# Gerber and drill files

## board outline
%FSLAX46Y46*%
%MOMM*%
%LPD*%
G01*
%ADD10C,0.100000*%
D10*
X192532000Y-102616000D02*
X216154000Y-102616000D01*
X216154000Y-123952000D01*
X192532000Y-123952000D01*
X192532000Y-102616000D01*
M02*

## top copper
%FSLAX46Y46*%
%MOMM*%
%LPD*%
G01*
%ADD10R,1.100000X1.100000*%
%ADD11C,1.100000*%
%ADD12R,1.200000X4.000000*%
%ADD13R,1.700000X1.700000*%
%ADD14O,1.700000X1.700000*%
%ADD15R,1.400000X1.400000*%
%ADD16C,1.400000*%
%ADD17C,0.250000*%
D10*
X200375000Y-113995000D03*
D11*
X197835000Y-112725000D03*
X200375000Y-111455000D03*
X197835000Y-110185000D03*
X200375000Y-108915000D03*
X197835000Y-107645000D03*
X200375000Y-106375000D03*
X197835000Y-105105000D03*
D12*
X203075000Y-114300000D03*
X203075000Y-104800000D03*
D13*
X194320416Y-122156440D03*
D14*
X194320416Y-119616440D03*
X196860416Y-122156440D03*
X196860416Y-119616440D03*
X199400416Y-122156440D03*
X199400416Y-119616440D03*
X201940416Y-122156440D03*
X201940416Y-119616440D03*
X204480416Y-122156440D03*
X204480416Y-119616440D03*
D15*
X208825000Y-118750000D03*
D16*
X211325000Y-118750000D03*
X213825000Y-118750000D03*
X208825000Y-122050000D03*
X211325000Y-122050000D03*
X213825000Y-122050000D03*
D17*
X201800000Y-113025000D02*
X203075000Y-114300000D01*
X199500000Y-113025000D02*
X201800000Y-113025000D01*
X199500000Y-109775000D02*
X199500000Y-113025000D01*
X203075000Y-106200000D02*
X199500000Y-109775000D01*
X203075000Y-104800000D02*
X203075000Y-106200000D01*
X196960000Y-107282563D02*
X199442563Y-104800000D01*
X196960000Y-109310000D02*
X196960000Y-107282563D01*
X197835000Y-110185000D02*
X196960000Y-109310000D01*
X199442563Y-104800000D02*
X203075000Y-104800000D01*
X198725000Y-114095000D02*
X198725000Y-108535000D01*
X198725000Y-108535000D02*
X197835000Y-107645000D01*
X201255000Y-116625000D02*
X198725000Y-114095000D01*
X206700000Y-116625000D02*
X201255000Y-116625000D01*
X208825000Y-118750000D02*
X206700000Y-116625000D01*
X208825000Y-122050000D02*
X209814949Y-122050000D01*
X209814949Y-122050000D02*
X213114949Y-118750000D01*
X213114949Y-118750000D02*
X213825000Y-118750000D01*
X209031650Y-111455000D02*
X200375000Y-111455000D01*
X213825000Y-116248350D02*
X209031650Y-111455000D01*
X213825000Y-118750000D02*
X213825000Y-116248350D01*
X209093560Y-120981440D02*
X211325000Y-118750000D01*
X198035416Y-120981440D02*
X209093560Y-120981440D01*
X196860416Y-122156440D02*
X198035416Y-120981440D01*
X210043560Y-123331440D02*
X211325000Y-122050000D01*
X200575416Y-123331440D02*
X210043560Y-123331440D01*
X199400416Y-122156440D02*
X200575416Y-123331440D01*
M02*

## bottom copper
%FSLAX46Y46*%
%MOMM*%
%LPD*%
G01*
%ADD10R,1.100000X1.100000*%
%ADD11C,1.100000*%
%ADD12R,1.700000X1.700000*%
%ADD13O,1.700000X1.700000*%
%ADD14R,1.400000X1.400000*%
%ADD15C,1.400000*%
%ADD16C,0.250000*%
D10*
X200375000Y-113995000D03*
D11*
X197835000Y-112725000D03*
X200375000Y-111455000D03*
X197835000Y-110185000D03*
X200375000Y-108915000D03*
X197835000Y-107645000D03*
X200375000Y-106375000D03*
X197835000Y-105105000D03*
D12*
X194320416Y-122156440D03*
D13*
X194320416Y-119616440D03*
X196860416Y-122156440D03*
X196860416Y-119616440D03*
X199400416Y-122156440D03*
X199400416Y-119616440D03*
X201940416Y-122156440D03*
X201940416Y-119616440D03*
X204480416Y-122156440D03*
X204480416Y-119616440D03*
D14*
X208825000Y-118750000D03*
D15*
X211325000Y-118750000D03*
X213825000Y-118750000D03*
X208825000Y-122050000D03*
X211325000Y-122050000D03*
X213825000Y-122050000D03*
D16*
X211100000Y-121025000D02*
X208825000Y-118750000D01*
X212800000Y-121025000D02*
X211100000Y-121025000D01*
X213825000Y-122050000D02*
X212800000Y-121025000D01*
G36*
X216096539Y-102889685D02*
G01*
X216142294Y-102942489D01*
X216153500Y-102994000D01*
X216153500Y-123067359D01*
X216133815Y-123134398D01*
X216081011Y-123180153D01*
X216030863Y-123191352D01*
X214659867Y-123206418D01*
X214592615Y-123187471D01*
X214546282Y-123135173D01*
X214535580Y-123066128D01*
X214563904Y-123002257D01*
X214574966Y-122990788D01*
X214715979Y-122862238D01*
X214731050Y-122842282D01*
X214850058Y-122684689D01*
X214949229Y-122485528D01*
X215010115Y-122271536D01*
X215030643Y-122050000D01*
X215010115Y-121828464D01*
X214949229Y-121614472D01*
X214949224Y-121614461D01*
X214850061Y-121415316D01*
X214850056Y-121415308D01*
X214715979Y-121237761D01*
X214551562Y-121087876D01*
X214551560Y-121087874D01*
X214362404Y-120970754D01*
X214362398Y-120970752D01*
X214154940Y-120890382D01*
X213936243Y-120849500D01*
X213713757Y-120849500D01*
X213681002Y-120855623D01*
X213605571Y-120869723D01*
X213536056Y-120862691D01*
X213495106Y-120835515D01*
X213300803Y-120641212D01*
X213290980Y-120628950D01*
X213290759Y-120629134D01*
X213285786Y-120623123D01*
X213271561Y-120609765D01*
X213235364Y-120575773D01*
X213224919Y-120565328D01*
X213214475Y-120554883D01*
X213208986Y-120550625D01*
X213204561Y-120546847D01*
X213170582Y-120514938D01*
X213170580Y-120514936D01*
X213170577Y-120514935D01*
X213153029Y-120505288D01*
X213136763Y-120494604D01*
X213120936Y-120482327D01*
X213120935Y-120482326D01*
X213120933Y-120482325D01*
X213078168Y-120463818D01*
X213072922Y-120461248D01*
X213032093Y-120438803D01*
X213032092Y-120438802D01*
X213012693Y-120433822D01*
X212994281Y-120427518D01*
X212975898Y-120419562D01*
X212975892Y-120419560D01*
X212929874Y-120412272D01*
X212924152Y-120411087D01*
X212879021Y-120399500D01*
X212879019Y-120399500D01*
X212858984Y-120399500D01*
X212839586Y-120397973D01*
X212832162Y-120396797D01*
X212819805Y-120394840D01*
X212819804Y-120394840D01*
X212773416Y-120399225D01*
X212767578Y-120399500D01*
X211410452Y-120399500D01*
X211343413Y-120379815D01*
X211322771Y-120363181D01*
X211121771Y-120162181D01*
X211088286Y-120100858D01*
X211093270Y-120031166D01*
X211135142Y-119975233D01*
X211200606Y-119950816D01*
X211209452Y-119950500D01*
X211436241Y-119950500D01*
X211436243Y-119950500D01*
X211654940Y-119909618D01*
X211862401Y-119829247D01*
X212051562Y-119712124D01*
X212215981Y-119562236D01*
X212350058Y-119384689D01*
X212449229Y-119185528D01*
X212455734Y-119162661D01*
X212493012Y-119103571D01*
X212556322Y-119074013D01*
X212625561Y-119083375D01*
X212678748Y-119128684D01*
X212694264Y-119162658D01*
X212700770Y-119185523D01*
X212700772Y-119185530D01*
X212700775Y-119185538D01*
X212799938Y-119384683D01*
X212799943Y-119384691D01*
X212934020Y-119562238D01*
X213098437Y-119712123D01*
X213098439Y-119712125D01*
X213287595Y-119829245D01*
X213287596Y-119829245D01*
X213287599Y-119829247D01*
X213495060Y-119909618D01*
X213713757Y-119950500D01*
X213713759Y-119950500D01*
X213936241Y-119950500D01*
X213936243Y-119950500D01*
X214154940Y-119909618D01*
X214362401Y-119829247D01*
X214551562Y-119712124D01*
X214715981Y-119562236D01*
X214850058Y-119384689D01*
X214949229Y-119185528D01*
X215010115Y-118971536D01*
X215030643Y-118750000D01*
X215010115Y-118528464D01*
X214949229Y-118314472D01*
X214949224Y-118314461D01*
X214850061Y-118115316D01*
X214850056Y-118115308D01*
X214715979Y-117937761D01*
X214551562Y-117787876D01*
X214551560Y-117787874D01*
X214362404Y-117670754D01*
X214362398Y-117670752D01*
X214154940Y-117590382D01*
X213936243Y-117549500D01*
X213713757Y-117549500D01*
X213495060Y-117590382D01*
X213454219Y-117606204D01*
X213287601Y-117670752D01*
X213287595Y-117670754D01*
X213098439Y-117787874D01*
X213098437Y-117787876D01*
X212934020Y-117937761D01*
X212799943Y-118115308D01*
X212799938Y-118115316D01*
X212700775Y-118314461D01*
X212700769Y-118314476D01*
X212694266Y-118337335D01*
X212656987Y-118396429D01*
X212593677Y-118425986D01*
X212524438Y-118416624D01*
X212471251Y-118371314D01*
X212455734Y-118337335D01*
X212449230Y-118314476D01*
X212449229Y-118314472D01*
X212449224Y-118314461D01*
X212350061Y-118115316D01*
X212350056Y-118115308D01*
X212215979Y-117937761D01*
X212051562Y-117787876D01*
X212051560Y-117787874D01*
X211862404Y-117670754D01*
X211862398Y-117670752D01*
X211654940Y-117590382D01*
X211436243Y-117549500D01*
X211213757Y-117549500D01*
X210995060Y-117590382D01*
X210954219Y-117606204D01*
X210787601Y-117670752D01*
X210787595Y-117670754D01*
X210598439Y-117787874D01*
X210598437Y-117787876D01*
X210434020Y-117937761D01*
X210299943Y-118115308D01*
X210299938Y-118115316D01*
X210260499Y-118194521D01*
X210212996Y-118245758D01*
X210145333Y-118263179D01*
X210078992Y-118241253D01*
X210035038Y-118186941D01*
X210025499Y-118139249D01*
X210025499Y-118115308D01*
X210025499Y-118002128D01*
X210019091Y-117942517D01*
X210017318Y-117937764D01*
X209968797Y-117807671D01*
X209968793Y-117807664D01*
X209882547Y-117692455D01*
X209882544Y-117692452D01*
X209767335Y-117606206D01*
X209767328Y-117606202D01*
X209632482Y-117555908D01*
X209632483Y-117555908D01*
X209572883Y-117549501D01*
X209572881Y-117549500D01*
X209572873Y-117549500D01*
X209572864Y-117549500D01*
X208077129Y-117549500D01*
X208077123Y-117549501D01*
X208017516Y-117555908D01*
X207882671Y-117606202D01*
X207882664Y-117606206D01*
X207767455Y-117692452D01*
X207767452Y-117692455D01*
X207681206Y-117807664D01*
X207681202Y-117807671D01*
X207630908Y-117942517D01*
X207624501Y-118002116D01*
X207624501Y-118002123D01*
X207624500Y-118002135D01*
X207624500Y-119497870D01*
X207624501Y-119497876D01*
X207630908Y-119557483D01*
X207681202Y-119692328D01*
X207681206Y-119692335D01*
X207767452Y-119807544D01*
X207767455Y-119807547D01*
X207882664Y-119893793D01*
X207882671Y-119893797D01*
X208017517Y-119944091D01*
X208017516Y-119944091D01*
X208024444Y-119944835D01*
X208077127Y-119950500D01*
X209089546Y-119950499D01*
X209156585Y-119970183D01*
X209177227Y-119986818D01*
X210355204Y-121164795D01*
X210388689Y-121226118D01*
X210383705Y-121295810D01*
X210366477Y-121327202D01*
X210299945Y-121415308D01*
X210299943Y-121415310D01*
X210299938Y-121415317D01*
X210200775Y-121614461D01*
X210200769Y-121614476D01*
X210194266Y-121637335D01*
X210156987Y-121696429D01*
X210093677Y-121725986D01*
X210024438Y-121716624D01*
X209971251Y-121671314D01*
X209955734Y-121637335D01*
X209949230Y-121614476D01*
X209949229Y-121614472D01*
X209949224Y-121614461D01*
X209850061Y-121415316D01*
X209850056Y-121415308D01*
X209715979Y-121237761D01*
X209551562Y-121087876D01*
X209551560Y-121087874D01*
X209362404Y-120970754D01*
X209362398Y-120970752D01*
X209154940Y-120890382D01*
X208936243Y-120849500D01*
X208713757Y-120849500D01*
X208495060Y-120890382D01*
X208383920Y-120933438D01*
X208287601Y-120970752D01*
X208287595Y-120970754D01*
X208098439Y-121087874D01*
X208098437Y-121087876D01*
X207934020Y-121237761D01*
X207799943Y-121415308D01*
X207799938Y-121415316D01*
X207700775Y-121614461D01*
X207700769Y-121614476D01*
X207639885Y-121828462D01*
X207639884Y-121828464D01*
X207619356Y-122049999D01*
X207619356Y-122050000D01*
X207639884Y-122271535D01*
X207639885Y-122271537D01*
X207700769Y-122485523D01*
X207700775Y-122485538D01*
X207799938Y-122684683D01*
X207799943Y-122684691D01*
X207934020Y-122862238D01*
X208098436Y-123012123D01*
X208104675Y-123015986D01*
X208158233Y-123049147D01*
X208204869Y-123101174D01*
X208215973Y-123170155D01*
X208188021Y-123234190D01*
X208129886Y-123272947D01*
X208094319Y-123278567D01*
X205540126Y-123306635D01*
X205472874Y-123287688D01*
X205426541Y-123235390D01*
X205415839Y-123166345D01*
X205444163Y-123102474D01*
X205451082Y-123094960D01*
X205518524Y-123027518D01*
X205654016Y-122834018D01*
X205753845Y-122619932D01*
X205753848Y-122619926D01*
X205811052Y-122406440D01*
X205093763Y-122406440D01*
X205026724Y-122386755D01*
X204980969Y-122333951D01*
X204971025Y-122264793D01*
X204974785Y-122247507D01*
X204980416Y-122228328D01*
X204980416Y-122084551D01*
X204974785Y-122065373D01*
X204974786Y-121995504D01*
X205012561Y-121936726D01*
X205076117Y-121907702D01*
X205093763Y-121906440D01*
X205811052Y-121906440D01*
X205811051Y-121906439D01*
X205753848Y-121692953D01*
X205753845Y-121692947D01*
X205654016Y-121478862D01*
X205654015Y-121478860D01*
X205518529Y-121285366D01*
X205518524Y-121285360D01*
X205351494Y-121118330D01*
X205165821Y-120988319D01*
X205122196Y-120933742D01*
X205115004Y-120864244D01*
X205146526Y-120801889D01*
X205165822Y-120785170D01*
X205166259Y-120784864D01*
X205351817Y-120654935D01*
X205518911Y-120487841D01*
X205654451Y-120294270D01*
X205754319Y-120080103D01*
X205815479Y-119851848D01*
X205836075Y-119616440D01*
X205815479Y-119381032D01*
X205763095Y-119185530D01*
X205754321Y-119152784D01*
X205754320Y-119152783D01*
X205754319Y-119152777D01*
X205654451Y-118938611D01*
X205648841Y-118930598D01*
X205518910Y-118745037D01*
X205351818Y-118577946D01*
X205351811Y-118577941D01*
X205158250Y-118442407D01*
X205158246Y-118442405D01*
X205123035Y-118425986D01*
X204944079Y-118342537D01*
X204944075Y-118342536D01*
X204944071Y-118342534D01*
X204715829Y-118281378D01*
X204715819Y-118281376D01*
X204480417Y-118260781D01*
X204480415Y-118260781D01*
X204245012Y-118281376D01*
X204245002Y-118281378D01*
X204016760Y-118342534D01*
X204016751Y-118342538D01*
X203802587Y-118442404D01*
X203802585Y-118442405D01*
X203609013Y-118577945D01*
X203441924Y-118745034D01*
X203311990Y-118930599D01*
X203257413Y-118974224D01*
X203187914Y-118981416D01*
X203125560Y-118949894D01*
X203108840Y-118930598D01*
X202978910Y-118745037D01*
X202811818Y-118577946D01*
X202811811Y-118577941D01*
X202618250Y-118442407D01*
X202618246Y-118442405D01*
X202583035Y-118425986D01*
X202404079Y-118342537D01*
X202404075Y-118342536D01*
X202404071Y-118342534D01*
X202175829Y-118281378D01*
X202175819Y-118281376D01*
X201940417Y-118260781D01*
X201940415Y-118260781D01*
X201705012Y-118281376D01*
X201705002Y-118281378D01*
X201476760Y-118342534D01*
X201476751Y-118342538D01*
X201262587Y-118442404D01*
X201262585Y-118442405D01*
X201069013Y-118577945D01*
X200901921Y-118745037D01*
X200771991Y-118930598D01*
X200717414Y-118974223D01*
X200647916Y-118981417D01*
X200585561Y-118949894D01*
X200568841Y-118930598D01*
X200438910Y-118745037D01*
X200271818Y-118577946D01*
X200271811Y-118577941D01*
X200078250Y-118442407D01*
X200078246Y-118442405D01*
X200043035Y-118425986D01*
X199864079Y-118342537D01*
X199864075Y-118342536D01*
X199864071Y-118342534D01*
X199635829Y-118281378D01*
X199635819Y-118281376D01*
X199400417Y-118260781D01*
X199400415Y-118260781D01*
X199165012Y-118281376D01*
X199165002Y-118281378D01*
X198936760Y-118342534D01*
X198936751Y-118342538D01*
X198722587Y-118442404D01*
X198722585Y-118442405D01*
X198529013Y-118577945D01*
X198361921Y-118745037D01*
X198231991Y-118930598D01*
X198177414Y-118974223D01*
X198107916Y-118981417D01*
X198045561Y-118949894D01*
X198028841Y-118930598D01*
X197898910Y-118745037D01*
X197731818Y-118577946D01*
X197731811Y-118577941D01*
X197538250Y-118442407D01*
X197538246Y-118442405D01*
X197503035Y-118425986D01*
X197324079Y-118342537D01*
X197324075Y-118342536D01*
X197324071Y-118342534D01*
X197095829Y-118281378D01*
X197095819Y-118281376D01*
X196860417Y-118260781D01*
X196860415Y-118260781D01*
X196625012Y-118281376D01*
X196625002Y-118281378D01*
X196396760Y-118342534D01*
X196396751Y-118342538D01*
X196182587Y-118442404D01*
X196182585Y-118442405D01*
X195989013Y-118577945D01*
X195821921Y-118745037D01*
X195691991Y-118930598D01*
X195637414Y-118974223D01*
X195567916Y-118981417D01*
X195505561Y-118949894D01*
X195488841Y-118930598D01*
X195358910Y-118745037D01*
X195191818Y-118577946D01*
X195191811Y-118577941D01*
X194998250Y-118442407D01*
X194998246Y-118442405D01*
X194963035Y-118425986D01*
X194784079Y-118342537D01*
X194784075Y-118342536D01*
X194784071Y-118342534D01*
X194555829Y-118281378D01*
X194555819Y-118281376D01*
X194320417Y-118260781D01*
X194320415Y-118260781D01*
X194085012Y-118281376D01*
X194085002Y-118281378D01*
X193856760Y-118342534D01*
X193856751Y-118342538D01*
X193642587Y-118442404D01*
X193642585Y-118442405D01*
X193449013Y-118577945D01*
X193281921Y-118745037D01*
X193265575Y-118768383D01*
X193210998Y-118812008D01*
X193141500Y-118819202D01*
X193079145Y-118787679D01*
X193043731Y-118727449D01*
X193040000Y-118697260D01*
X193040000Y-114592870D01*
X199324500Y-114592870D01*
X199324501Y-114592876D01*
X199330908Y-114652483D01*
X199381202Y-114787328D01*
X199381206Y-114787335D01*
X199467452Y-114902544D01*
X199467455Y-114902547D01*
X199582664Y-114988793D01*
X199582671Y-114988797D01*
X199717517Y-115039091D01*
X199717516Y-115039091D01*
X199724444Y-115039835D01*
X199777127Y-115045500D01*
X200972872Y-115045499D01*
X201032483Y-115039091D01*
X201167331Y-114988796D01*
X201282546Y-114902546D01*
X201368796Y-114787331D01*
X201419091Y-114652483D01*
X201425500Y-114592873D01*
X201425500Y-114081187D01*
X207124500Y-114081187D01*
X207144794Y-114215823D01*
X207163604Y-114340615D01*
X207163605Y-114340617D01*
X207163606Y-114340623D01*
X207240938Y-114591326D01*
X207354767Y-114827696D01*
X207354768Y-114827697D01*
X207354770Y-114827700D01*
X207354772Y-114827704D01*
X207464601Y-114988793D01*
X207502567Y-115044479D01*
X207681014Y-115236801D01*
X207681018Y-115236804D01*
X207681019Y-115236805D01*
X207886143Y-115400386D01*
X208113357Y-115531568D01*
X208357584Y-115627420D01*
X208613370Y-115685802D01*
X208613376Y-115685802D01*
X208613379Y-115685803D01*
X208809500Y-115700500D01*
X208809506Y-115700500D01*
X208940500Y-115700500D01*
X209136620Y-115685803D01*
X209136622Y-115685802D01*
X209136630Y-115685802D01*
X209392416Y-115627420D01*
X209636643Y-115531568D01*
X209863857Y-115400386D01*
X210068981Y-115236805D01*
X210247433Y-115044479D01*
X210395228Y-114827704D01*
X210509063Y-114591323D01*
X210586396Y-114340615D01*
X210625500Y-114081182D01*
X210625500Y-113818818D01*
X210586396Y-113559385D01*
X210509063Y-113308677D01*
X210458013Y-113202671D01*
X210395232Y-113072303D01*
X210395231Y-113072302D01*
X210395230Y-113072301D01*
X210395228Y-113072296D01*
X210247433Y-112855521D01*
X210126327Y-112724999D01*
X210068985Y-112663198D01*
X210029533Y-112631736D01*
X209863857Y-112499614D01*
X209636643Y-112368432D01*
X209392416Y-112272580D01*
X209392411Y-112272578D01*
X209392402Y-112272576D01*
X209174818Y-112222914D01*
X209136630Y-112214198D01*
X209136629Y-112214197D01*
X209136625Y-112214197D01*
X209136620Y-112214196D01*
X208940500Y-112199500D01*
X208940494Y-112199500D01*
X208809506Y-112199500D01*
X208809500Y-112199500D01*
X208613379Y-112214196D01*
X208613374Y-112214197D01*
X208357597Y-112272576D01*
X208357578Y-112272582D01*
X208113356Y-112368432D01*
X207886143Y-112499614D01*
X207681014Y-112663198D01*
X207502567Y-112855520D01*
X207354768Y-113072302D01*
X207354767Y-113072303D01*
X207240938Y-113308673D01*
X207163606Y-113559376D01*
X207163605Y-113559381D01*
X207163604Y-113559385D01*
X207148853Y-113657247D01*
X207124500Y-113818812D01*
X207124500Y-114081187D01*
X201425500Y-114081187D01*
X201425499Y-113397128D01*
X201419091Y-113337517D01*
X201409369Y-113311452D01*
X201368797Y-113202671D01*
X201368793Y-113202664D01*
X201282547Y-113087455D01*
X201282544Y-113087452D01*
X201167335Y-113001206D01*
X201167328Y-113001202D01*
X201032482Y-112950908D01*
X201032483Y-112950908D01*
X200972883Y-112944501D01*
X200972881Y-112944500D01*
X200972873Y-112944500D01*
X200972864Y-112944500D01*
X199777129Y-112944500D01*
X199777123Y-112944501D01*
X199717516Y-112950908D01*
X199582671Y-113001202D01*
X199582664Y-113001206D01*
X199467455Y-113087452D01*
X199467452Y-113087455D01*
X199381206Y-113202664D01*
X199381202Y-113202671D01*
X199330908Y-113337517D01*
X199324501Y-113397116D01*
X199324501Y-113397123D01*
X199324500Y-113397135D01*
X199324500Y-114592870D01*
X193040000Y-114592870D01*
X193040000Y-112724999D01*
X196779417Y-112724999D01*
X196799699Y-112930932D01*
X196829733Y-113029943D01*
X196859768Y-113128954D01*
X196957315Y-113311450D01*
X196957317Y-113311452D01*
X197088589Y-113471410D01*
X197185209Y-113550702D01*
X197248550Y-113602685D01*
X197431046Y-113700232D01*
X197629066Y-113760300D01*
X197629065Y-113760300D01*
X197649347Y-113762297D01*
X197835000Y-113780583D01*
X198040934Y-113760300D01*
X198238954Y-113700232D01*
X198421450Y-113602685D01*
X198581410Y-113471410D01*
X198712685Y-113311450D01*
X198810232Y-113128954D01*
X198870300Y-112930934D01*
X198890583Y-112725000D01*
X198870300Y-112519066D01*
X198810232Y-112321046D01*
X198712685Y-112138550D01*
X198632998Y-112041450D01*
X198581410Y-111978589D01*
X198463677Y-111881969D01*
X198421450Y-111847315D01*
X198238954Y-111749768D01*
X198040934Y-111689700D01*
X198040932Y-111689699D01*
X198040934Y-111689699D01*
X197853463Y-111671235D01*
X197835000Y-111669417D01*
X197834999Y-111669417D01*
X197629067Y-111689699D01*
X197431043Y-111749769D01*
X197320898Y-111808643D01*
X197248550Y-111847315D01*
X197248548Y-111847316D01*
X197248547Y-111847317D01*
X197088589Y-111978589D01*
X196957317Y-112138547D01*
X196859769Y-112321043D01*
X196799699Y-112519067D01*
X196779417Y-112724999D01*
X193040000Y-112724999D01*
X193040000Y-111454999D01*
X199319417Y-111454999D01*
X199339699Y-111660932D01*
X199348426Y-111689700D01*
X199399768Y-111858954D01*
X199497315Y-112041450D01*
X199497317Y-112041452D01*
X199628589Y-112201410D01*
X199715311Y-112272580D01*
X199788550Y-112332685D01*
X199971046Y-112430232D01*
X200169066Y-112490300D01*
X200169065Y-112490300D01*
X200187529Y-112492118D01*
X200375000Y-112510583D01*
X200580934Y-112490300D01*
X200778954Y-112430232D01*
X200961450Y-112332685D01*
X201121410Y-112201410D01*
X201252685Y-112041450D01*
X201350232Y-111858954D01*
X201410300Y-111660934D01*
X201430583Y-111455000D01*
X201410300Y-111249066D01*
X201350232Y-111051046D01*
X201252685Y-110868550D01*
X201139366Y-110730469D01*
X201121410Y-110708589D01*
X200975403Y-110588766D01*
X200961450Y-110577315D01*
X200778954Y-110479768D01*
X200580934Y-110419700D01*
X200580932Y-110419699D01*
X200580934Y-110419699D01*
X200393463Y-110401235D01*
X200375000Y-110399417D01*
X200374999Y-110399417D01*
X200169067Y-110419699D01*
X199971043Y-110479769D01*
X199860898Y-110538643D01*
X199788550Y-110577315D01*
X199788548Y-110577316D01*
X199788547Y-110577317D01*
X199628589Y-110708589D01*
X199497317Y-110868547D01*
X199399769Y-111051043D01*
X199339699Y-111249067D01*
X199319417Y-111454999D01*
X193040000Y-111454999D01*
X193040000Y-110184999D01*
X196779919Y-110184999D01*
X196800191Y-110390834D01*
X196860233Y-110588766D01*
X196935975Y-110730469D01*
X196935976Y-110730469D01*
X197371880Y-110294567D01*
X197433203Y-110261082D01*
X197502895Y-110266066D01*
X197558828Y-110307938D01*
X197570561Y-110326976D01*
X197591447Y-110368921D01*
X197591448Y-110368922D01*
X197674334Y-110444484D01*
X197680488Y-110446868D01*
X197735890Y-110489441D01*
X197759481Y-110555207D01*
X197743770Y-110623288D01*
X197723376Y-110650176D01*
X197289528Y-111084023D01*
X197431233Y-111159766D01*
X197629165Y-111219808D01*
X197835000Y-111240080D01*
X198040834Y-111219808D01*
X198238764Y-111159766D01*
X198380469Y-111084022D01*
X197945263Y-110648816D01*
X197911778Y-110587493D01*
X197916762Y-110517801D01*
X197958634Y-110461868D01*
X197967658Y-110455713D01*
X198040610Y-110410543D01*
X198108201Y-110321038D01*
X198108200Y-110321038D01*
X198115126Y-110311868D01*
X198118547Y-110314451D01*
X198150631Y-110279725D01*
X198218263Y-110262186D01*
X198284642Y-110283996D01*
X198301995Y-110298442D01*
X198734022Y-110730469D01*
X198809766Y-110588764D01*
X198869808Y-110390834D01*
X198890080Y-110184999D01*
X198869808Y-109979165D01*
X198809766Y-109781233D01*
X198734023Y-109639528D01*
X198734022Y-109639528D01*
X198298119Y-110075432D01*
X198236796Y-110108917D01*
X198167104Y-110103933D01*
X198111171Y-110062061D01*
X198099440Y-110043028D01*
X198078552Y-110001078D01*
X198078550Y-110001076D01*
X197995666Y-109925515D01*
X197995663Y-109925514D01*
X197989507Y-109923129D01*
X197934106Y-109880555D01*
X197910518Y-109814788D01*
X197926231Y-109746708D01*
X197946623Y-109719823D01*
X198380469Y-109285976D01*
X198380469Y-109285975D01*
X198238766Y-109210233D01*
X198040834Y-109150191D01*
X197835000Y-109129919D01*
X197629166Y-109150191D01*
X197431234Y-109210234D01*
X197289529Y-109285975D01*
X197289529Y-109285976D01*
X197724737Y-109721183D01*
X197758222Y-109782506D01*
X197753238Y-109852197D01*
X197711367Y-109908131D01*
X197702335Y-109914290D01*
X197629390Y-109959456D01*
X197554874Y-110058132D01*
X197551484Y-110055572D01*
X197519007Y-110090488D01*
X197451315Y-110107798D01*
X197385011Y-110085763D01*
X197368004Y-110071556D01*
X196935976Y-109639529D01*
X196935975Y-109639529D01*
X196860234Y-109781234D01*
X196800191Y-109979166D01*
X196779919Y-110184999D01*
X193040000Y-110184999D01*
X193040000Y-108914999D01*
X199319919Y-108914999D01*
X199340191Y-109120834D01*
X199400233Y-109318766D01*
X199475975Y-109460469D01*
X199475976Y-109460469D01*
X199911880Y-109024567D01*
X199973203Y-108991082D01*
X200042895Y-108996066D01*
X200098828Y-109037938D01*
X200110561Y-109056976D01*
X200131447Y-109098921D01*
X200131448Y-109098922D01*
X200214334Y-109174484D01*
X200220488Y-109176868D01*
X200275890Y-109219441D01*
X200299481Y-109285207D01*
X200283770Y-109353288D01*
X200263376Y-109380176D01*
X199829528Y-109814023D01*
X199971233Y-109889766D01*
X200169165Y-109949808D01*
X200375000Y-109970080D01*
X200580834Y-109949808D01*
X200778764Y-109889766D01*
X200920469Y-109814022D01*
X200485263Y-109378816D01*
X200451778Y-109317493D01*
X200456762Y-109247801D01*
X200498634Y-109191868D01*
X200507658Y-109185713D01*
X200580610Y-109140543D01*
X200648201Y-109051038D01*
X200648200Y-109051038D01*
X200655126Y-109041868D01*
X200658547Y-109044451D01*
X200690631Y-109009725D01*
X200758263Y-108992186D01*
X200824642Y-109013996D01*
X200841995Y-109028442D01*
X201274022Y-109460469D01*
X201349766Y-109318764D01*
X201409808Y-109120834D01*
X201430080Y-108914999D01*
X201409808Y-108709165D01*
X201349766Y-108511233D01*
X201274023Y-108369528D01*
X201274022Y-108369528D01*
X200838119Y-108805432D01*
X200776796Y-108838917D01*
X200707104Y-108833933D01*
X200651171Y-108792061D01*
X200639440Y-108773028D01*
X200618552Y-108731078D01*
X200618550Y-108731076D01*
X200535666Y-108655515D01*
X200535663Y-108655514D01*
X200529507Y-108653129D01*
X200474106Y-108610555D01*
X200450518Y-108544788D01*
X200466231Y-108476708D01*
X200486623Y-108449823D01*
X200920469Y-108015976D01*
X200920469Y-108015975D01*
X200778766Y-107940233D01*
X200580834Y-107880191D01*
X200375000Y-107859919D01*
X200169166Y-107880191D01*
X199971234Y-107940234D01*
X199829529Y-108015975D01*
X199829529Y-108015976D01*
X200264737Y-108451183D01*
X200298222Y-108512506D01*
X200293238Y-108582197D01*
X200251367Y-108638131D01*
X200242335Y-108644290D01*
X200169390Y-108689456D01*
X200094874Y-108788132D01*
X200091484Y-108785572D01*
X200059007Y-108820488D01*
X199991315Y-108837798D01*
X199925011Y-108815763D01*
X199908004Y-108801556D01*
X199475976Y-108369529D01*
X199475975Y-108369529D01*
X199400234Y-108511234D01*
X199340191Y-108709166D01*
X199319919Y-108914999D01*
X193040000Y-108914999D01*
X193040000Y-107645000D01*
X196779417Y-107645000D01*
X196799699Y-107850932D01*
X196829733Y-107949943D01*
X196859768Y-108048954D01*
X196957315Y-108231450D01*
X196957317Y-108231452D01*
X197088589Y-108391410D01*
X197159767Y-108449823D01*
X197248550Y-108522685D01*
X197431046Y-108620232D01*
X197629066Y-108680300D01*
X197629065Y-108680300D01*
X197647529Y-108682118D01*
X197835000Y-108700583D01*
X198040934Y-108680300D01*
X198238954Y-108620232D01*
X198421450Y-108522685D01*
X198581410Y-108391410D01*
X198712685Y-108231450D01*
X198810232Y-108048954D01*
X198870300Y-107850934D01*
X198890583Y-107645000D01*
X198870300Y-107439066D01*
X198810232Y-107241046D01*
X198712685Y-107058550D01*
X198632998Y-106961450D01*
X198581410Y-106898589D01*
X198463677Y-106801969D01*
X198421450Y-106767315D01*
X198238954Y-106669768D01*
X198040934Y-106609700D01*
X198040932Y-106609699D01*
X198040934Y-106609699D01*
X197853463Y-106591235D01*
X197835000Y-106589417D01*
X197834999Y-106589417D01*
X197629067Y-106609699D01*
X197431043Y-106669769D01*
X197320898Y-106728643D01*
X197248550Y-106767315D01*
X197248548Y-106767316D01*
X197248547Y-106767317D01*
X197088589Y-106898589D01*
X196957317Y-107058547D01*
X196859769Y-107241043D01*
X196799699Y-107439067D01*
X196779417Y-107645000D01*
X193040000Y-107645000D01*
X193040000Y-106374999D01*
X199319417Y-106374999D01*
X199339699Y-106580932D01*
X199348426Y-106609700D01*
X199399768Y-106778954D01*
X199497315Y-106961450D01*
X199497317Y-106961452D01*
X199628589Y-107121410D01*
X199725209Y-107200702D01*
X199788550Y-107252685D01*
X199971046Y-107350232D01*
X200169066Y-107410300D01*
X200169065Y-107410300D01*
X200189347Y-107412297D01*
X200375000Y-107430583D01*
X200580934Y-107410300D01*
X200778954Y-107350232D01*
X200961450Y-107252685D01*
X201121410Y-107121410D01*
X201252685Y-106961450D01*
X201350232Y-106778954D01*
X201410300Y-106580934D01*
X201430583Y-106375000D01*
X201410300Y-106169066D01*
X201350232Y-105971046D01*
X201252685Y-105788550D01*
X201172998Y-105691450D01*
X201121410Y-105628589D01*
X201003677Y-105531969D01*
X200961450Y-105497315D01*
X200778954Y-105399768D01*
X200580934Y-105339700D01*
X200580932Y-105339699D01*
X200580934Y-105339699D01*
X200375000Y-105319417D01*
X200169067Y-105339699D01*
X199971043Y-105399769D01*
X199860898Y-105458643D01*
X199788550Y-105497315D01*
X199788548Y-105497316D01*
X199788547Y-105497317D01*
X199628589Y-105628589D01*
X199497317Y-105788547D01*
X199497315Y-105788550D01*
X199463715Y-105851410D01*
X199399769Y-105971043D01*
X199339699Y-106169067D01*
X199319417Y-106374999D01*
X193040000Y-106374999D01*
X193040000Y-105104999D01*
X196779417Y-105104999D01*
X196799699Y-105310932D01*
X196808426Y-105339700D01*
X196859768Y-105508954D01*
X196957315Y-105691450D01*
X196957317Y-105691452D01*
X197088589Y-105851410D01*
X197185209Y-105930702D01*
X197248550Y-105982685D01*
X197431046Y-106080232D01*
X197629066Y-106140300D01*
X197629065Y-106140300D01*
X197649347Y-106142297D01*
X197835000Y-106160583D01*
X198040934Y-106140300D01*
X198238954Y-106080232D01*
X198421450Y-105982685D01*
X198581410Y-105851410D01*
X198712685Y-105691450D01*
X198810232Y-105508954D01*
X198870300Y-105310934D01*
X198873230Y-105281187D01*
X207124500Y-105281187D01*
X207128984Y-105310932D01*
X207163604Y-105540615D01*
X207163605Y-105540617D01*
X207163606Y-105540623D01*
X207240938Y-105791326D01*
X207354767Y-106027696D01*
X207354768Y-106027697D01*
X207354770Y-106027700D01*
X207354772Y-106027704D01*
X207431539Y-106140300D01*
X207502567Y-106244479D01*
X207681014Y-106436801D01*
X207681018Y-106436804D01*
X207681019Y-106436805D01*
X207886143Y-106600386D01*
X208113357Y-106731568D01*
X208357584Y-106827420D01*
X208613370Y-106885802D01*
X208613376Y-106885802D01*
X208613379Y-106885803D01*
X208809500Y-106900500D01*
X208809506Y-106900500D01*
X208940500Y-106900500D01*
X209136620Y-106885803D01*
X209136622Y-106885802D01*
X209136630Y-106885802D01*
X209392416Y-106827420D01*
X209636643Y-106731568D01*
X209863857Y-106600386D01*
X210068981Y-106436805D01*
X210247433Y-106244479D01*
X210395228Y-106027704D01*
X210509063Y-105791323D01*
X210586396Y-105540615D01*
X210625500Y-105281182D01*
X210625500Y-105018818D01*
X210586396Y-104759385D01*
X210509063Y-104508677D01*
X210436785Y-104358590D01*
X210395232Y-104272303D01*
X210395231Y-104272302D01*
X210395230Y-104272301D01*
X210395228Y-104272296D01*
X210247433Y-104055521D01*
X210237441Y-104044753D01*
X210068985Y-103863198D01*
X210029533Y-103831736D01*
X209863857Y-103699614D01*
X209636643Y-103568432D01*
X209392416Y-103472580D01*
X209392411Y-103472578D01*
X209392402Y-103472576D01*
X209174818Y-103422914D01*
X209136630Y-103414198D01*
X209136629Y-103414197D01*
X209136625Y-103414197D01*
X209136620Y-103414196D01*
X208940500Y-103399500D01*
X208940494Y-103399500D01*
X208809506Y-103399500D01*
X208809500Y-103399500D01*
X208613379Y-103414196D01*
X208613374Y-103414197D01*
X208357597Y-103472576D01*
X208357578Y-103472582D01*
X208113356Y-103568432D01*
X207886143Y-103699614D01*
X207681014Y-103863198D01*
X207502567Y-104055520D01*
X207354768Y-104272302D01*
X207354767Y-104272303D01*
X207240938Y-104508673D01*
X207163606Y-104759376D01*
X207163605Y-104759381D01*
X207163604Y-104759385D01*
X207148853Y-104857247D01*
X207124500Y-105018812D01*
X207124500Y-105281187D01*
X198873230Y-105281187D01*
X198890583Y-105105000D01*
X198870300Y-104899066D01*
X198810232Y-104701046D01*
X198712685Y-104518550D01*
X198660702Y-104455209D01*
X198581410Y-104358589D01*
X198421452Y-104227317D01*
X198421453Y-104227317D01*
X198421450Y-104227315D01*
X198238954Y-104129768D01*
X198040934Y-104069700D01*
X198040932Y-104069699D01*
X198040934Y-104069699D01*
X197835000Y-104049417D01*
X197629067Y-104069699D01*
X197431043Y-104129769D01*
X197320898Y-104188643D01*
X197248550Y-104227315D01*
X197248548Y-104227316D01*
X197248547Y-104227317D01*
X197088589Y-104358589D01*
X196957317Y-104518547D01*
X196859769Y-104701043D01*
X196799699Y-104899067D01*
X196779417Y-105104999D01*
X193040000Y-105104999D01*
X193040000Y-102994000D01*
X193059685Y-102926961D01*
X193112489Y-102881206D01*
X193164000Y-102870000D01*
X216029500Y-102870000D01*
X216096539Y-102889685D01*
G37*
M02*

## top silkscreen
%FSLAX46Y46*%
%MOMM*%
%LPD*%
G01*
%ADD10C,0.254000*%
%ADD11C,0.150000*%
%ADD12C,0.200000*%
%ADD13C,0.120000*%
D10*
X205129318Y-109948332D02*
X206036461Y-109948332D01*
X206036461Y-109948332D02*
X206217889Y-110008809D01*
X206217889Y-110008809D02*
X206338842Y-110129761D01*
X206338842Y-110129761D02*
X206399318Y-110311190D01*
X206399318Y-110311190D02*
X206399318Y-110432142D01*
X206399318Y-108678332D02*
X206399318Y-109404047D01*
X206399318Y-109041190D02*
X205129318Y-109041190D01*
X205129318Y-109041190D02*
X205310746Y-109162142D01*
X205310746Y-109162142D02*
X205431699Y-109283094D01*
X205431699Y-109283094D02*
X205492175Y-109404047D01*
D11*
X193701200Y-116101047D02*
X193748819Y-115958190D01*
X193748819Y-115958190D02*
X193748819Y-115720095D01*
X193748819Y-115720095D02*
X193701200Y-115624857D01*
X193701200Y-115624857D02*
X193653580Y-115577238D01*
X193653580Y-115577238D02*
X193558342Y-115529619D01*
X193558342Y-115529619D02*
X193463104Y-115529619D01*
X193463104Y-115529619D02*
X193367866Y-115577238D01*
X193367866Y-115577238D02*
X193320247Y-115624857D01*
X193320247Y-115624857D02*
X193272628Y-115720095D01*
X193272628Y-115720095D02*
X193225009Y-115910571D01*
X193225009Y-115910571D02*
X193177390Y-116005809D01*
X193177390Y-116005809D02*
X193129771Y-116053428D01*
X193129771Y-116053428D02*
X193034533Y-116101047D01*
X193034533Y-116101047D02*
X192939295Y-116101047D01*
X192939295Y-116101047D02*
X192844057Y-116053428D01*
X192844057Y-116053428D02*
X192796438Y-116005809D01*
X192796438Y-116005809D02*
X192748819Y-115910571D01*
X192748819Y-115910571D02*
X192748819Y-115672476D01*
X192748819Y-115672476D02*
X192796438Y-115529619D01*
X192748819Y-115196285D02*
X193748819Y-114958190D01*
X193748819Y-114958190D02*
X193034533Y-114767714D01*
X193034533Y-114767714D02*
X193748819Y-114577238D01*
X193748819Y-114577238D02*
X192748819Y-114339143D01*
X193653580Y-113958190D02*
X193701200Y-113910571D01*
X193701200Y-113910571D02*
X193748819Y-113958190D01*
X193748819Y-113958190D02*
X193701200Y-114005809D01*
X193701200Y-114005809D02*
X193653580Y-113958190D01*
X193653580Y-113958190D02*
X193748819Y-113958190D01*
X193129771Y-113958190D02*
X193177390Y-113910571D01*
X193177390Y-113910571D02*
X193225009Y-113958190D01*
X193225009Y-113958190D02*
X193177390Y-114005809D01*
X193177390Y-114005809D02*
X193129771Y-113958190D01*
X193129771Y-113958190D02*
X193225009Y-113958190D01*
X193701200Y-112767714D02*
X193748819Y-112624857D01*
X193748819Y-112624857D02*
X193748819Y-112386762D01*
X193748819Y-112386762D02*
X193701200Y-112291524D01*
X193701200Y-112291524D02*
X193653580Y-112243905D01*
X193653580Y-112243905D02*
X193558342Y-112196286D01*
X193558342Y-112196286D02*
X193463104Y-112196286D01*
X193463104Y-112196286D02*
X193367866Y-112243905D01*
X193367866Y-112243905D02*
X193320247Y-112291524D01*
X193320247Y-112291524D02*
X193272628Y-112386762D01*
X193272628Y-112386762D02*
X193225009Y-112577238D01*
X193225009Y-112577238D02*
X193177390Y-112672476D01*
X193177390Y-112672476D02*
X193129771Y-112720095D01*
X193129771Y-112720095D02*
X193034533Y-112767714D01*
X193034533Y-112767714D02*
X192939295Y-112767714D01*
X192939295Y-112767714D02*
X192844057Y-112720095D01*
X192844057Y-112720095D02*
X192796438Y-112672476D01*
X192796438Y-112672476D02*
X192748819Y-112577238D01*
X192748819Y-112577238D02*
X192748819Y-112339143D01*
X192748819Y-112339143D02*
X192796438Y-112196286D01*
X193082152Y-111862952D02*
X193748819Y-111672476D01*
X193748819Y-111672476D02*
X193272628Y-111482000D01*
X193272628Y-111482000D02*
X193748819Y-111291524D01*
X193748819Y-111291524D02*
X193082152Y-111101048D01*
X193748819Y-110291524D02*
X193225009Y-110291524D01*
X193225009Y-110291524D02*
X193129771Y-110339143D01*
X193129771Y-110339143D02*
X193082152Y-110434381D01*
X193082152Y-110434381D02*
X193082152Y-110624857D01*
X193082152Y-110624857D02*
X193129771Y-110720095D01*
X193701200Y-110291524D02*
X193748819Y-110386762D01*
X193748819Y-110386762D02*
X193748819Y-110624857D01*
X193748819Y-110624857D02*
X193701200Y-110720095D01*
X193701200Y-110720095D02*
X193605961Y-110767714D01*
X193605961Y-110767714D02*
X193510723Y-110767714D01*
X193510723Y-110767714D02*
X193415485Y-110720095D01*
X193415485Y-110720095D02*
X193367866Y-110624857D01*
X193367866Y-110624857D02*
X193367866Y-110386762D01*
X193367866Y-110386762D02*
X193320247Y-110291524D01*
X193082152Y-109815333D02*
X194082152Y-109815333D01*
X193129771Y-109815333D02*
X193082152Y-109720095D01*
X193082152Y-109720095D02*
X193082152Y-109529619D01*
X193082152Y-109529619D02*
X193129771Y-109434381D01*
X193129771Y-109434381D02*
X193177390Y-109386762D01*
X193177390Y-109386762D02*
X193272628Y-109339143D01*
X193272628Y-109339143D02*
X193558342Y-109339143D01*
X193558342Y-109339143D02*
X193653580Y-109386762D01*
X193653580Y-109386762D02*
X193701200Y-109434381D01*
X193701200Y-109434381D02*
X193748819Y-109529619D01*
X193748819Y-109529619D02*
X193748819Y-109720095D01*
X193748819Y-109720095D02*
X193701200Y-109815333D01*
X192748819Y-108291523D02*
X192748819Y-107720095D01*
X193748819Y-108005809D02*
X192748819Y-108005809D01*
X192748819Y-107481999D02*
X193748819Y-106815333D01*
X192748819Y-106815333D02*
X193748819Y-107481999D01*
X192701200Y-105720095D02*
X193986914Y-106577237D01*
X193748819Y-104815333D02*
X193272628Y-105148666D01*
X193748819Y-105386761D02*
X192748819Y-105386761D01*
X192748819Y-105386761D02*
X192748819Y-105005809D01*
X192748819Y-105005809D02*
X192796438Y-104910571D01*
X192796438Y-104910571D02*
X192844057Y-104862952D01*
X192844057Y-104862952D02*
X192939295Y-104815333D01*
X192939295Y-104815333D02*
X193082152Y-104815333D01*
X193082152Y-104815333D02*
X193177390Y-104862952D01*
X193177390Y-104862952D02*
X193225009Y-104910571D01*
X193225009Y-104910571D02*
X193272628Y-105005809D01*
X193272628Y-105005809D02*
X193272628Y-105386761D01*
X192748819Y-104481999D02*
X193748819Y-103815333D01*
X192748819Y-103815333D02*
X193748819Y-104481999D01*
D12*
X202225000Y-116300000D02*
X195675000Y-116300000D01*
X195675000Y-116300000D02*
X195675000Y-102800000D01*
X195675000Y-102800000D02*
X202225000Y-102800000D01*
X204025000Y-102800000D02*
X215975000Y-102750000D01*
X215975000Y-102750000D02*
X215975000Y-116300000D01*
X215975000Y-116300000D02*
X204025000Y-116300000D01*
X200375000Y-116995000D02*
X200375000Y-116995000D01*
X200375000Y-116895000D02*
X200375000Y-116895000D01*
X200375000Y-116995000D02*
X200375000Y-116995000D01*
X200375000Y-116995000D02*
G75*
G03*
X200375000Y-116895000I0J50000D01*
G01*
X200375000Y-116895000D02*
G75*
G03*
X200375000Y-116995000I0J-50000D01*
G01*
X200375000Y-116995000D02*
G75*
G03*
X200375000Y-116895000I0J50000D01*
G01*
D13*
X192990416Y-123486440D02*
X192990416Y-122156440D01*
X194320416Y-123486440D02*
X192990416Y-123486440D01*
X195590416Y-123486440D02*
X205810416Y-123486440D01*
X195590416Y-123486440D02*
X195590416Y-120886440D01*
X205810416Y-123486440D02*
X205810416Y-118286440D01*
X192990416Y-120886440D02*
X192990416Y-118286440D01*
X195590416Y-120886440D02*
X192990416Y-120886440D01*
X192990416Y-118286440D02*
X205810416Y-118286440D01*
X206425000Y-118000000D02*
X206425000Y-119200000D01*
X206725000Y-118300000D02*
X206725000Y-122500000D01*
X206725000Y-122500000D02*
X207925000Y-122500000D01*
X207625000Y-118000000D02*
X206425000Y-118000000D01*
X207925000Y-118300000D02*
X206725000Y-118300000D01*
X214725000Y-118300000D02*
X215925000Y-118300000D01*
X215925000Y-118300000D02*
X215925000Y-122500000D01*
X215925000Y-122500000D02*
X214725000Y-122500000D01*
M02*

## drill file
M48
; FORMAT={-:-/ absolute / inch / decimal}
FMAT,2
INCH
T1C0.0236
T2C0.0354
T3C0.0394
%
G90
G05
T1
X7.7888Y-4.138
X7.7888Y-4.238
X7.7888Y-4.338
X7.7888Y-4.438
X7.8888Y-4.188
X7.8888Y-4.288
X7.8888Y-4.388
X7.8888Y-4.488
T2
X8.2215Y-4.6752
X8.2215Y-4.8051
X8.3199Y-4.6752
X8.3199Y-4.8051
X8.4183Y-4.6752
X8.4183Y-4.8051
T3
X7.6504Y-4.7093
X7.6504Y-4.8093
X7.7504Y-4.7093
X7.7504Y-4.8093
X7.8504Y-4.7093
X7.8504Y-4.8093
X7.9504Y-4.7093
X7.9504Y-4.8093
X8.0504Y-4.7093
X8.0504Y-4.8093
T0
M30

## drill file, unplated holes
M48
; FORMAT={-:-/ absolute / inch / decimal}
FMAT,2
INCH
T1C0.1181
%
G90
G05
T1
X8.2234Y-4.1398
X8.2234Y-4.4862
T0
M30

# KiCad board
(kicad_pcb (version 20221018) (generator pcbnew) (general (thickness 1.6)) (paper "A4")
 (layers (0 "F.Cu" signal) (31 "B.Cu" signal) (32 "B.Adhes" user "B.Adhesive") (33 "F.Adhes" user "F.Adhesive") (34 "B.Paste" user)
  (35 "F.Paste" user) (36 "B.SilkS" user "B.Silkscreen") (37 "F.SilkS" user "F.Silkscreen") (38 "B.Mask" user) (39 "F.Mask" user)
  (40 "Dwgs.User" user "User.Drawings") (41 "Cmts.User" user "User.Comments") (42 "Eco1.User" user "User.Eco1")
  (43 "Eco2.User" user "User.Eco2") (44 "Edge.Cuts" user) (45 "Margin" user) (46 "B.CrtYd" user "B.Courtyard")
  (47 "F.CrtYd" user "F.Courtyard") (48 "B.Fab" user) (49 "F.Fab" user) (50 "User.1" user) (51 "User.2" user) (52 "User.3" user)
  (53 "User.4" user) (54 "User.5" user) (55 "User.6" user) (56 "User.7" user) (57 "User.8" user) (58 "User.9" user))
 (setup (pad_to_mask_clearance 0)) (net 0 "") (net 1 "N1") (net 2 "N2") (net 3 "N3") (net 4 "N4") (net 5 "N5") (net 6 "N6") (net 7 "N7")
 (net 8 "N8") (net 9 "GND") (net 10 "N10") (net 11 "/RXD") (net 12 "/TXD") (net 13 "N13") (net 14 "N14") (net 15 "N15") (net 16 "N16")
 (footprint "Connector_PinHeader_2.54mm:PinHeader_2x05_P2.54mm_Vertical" (layer "F.Cu") (at 194.320416 122.15644 90)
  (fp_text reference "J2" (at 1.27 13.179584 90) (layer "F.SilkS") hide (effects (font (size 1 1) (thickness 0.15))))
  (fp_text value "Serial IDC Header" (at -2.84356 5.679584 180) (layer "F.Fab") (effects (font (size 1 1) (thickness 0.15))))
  (fp_line (start -1.33 -1.33) (end 0 -1.33) (stroke (width 0.12) (type solid)) (layer "F.SilkS"))
  (fp_line (start -1.33 0) (end -1.33 -1.33) (stroke (width 0.12) (type solid)) (layer "F.SilkS"))
  (fp_line (start -1.33 1.27) (end -1.33 11.49) (stroke (width 0.12) (type solid)) (layer "F.SilkS"))
  (fp_line (start -1.33 1.27) (end 1.27 1.27) (stroke (width 0.12) (type solid)) (layer "F.SilkS"))
  (fp_line (start -1.33 11.49) (end 3.87 11.49) (stroke (width 0.12) (type solid)) (layer "F.SilkS"))
  (fp_line (start 1.27 -1.33) (end 3.87 -1.33) (stroke (width 0.12) (type solid)) (layer "F.SilkS"))
  (fp_line (start 1.27 1.27) (end 1.27 -1.33) (stroke (width 0.12) (type solid)) (layer "F.SilkS"))
  (fp_line (start 3.87 -1.33) (end 3.87 11.49) (stroke (width 0.12) (type solid)) (layer "F.SilkS"))
  (pad "1" thru_hole rect (at 0 0 90) (size 1.7 1.7) (drill 1) (layers "*.Cu" "*.Mask") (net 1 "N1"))
  (pad "2" thru_hole oval (at 2.54 0 90) (size 1.7 1.7) (drill 1) (layers "*.Cu" "*.Mask") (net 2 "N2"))
  (pad "3" thru_hole oval (at 0 2.54 90) (size 1.7 1.7) (drill 1) (layers "*.Cu" "*.Mask") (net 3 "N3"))
  (pad "4" thru_hole oval (at 2.54 2.54 90) (size 1.7 1.7) (drill 1) (layers "*.Cu" "*.Mask") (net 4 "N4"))
  (pad "5" thru_hole oval (at 0 5.08 90) (size 1.7 1.7) (drill 1) (layers "*.Cu" "*.Mask") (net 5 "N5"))
  (pad "6" thru_hole oval (at 2.54 5.08 90) (size 1.7 1.7) (drill 1) (layers "*.Cu" "*.Mask") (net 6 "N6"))
  (pad "7" thru_hole oval (at 0 7.62 90) (size 1.7 1.7) (drill 1) (layers "*.Cu" "*.Mask") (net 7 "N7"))
  (pad "8" thru_hole oval (at 2.54 7.62 90) (size 1.7 1.7) (drill 1) (layers "*.Cu" "*.Mask") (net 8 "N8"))
  (pad "9" thru_hole oval (at 0 10.16 90) (size 1.7 1.7) (drill 1) (layers "*.Cu" "*.Mask") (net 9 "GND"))
  (pad "10" thru_hole oval (at 2.54 10.16 90) (size 1.7 1.7) (drill 1) (layers "*.Cu" "*.Mask") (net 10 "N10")))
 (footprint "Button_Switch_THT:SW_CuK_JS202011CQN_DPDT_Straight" (layer "F.Cu") (at 208.825 118.75)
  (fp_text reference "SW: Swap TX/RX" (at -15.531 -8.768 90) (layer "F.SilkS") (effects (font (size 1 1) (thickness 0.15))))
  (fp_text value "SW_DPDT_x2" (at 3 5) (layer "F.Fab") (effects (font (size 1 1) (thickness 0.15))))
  (fp_line (start -2.4 -0.75) (end -2.4 0.45) (stroke (width 0.12) (type solid)) (layer "F.SilkS"))
  (fp_line (start -2.1 -0.45) (end -2.1 3.75) (stroke (width 0.12) (type solid)) (layer "F.SilkS"))
  (fp_line (start -2.1 3.75) (end -0.9 3.75) (stroke (width 0.12) (type solid)) (layer "F.SilkS"))
  (fp_line (start -1.2 -0.75) (end -2.4 -0.75) (stroke (width 0.12) (type solid)) (layer "F.SilkS"))
  (fp_line (start -0.9 -0.45) (end -2.1 -0.45) (stroke (width 0.12) (type solid)) (layer "F.SilkS"))
  (fp_line (start 5.9 -0.45) (end 7.1 -0.45) (stroke (width 0.12) (type solid)) (layer "F.SilkS"))
  (fp_line (start 7.1 -0.45) (end 7.1 3.75) (stroke (width 0.12) (type solid)) (layer "F.SilkS"))
  (fp_line (start 7.1 3.75) (end 5.9 3.75) (stroke (width 0.12) (type solid)) (layer "F.SilkS"))
  (pad "1" thru_hole rect (at 0 0) (size 1.4 1.4) (drill 0.9) (layers "*.Cu" "*.Mask") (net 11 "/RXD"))
  (pad "2" thru_hole circle (at 2.5 0) (size 1.4 1.4) (drill 0.9) (layers "*.Cu" "*.Mask") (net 3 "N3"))
  (pad "3" thru_hole circle (at 5 0) (size 1.4 1.4) (drill 0.9) (layers "*.Cu" "*.Mask") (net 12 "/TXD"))
  (pad "4" thru_hole circle (at 0 3.3) (size 1.4 1.4) (drill 0.9) (layers "*.Cu" "*.Mask") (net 12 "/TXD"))
  (pad "5" thru_hole circle (at 2.5 3.3) (size 1.4 1.4) (drill 0.9) (layers "*.Cu" "*.Mask") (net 5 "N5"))
  (pad "6" thru_hole circle (at 5 3.3) (size 1.4 1.4) (drill 0.9) (layers "*.Cu" "*.Mask") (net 11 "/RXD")))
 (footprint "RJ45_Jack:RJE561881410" (layer "F.Cu") (at 200.375 113.995 90)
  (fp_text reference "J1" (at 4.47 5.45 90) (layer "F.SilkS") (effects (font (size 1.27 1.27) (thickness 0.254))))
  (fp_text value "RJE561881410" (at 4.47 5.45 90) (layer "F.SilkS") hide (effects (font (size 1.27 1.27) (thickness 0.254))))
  (fp_line (start -3 0) (end -3 0) (stroke (width 0.2) (type solid)) (layer "F.SilkS"))
  (fp_line (start -3 0) (end -3 0) (stroke (width 0.2) (type solid)) (layer "F.SilkS"))
  (fp_line (start -2.9 0) (end -2.9 0) (stroke (width 0.2) (type solid)) (layer "F.SilkS"))
  (fp_line (start -2.305 -4.7) (end 11.195 -4.7) (stroke (width 0.2) (type solid)) (layer "F.SilkS"))
  (fp_line (start -2.305 1.85) (end -2.305 -4.7) (stroke (width 0.2) (type solid)) (layer "F.SilkS"))
  (fp_line (start -2.305 15.6) (end -2.305 3.65) (stroke (width 0.2) (type solid)) (layer "F.SilkS"))
  (fp_line (start 11.195 -4.7) (end 11.195 1.85) (stroke (width 0.2) (type solid)) (layer "F.SilkS"))
  (fp_line (start 11.195 3.65) (end 11.245 15.6) (stroke (width 0.2) (type solid)) (layer "F.SilkS"))
  (fp_line (start 11.245 15.6) (end -2.305 15.6) (stroke (width 0.2) (type solid)) (layer "F.SilkS"))
  (fp_arc (start -3 0) (mid -2.95 -0.05) (end -2.9 0) (stroke (width 0.2) (type solid)) (layer "F.SilkS"))
  (fp_arc (start -2.9 0) (mid -2.95 0.05) (end -3 0) (stroke (width 0.2) (type solid)) (layer "F.SilkS"))
  (fp_arc (start -2.9 0) (mid -2.95 0.05) (end -3 0) (stroke (width 0.2) (type solid)) (layer "F.SilkS"))
  (pad "" np_thru_hole circle (at 0.045 8.5 90) (size 3 3) (drill 3) (layers "*.Cu" "*.Mask"))
  (pad "" np_thru_hole circle (at 8.845 8.5 90) (size 3 3) (drill 3) (layers "*.Cu" "*.Mask"))
  (pad "1" thru_hole rect (at 0 0 90) (size 1.1 1.1) (drill 0.6) (layers "*.Cu" "*.Mask") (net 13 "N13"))
  (pad "2" thru_hole circle (at 1.27 -2.54 90) (size 1.1 1.1) (drill 0.6) (layers "*.Cu" "*.Mask") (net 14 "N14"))
  (pad "3" thru_hole circle (at 2.54 0 90) (size 1.1 1.1) (drill 0.6) (layers "*.Cu" "*.Mask") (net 12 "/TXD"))
  (pad "4" thru_hole circle (at 3.81 -2.54 90) (size 1.1 1.1) (drill 0.6) (layers "*.Cu" "*.Mask") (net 9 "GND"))
  (pad "5" thru_hole circle (at 5.08 0 90) (size 1.1 1.1) (drill 0.6) (layers "*.Cu" "*.Mask") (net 9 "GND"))
  (pad "6" thru_hole circle (at 6.35 -2.54 90) (size 1.1 1.1) (drill 0.6) (layers "*.Cu" "*.Mask") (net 11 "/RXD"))
  (pad "7" thru_hole circle (at 7.62 0 90) (size 1.1 1.1) (drill 0.6) (layers "*.Cu" "*.Mask") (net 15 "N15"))
  (pad "8" thru_hole circle (at 8.89 -2.54 90) (size 1.1 1.1) (drill 0.6) (layers "*.Cu" "*.Mask") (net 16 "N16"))
  (pad "G1" smd rect (at -0.305 2.7 180) (size 1.2 4) (layers "F.Cu" "F.Paste" "F.Mask") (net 9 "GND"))
  (pad "G2" smd rect (at 9.195 2.7 180) (size 1.2 4) (layers "F.Cu" "F.Paste" "F.Mask") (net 9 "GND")))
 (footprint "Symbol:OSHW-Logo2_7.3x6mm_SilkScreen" (layer "B.Cu") (at 211.836 108.966 180)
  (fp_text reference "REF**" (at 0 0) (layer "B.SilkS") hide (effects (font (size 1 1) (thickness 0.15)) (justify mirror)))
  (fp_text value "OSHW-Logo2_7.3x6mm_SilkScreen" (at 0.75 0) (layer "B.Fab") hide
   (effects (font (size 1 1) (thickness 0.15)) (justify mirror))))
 (gr_rect (start 192.532 102.616) (end 216.154 123.952) (stroke (width 0.1) (type default)) (fill none) (layer "Edge.Cuts"))
 (segment (start 208.825 122.05) (end 209.814949 122.05) (width 0.25) (layer "F.Cu") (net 12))
 (segment (start 213.825 118.75) (end 213.825 116.24835) (width 0.25) (layer "F.Cu") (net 12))
 (segment (start 209.03165 111.455) (end 200.375 111.455) (width 0.25) (layer "F.Cu") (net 12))
 (segment (start 213.825 116.24835) (end 209.03165 111.455) (width 0.25) (layer "F.Cu") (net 12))
 (segment (start 209.814949 122.05) (end 213.114949 118.75) (width 0.25) (layer "F.Cu") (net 12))
 (segment (start 213.114949 118.75) (end 213.825 118.75) (width 0.25) (layer "F.Cu") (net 12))
 (segment (start 201.8 113.025) (end 203.075 114.3) (width 0.25) (layer "F.Cu") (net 9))
 (segment (start 203.075 106.2) (end 199.5 109.775) (width 0.25) (layer "F.Cu") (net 9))
 (segment (start 203.075 104.8) (end 203.075 106.2) (width 0.25) (layer "F.Cu") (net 9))
 (segment (start 199.5 113.025) (end 201.8 113.025) (width 0.25) (layer "F.Cu") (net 9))
 (segment (start 199.5 109.775) (end 199.5 113.025) (width 0.25) (layer "F.Cu") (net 9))
 (segment (start 196.96 109.31) (end 196.96 107.282563) (width 0.25) (layer "F.Cu") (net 9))
 (segment (start 197.835 110.185) (end 196.96 109.31) (width 0.25) (layer "F.Cu") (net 9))
 (segment (start 199.442563 104.8) (end 203.075 104.8) (width 0.25) (layer "F.Cu") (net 9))
 (segment (start 196.96 107.282563) (end 199.442563 104.8) (width 0.25) (layer "F.Cu") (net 9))
 (segment (start 198.725 114.095) (end 198.725 108.535) (width 0.25) (layer "F.Cu") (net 11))
 (segment (start 198.725 108.535) (end 197.835 107.645) (width 0.25) (layer "F.Cu") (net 11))
 (segment (start 206.7 116.625) (end 201.255 116.625) (width 0.25) (layer "F.Cu") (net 11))
 (segment (start 201.255 116.625) (end 198.725 114.095) (width 0.25) (layer "F.Cu") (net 11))
 (segment (start 208.825 118.75) (end 206.7 116.625) (width 0.25) (layer "F.Cu") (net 11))
 (segment (start 213.825 122.05) (end 212.8 121.025) (width 0.25) (layer "B.Cu") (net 11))
 (segment (start 212.8 121.025) (end 211.1 121.025) (width 0.25) (layer "B.Cu") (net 11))
 (segment (start 211.1 121.025) (end 208.825 118.75) (width 0.25) (layer "B.Cu") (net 11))
 (segment (start 198.035416 120.98144) (end 209.09356 120.98144) (width 0.25) (layer "F.Cu") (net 3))
 (segment (start 209.09356 120.98144) (end 211.325 118.75) (width 0.25) (layer "F.Cu") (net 3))
 (segment (start 196.860416 122.15644) (end 198.035416 120.98144) (width 0.25) (layer "F.Cu") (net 3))
 (segment (start 210.04356 123.33144) (end 211.325 122.05) (width 0.25) (layer "F.Cu") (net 5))
 (segment (start 200.575416 123.33144) (end 210.04356 123.33144) (width 0.25) (layer "F.Cu") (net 5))
 (segment (start 199.400416 122.15644) (end 200.575416 123.33144) (width 0.25) (layer "F.Cu") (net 5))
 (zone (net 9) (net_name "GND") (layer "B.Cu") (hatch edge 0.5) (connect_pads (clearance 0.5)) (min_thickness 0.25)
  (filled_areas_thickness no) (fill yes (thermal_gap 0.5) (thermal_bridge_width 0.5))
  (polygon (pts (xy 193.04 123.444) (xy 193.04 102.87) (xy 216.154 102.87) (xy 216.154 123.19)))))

